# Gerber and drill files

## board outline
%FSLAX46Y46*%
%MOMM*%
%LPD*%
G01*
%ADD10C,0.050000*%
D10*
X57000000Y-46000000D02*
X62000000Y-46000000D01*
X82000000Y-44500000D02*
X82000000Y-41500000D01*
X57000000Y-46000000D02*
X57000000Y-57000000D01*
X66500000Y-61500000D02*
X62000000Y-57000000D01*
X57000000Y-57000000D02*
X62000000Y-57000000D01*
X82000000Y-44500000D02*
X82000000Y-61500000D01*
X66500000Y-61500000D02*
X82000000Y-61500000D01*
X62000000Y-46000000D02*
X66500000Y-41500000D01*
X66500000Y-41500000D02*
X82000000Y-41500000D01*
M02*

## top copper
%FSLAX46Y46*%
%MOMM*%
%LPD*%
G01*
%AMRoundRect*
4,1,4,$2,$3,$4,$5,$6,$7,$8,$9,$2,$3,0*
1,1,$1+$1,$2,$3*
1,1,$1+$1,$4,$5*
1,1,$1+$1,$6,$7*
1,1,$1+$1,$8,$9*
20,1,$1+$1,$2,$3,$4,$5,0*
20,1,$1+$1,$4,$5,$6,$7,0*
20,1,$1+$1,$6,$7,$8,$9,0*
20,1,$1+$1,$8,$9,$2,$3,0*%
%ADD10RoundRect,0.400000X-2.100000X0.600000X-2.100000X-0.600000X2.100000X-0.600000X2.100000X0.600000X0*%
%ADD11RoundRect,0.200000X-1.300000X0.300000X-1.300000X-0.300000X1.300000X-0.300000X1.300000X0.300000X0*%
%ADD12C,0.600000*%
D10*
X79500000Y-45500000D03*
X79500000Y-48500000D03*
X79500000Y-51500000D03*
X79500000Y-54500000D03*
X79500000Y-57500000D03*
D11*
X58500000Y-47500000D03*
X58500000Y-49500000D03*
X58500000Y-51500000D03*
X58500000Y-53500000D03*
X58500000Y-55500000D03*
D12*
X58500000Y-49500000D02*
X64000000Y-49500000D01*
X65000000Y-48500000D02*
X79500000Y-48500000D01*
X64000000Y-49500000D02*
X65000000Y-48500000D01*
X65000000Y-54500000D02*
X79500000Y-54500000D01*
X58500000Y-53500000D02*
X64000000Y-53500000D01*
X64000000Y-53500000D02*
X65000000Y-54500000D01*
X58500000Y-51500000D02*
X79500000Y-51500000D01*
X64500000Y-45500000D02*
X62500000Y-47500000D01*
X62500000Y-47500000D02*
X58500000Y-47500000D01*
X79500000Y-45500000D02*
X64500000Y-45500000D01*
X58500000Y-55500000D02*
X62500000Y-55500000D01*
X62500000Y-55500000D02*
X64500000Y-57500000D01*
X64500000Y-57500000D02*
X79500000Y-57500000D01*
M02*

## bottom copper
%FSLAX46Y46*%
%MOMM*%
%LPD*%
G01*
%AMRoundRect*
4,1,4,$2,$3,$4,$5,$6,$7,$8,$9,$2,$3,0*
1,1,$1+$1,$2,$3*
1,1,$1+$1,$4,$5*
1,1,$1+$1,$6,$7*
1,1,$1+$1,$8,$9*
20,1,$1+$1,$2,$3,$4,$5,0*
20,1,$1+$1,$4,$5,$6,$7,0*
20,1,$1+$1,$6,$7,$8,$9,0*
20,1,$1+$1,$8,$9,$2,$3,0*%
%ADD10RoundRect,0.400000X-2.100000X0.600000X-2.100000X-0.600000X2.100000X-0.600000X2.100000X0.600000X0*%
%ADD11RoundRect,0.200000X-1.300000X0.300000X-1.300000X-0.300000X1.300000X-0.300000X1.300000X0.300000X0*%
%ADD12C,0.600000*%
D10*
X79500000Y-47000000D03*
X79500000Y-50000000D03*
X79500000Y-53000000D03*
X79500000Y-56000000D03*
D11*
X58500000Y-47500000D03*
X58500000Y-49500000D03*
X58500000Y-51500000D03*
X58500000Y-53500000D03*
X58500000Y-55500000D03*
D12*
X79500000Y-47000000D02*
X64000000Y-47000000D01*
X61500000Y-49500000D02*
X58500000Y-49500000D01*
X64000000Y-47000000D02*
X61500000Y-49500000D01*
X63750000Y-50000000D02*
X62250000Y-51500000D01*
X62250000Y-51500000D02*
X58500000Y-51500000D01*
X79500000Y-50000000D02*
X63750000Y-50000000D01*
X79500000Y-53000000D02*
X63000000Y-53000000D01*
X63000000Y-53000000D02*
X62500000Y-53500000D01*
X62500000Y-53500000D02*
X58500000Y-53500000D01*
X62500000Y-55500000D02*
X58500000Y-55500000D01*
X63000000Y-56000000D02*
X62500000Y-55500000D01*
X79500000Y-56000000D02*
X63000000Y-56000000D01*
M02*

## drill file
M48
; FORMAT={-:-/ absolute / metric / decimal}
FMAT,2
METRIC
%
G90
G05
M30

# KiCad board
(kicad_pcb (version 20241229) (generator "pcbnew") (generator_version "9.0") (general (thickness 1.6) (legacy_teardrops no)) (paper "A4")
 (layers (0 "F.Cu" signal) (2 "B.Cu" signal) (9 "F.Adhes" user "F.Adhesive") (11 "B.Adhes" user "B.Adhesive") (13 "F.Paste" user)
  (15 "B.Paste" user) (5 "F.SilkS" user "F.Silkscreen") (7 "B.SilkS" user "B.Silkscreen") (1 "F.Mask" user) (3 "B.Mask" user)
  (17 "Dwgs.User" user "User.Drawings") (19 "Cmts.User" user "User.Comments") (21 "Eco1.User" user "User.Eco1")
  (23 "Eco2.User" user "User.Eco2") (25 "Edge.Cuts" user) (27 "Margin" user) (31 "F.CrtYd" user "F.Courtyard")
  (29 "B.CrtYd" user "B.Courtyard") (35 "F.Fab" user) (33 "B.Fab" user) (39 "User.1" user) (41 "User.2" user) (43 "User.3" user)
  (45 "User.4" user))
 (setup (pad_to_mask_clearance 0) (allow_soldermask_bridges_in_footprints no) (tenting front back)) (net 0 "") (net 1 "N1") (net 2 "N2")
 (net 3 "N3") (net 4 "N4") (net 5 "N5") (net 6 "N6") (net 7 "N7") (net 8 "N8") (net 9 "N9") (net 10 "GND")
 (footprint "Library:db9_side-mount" (layer "F.Cu") (at 79.5 51.5 -90)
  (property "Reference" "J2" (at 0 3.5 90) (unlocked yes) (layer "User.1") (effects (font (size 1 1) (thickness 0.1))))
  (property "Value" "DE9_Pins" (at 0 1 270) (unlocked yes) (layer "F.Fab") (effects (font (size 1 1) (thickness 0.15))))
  (pad "1" smd roundrect (at -6 0 270) (size 2 5) (layers "F.Cu" "F.Mask" "F.Paste") (roundrect_rratio 0.2) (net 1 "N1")
   (thermal_bridge_angle 45))
  (pad "2" smd roundrect (at -3 0 270) (size 2 5) (layers "F.Cu" "F.Mask" "F.Paste") (roundrect_rratio 0.2) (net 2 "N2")
   (thermal_bridge_angle 45))
  (pad "3" smd roundrect (at 0 0 270) (size 2 5) (layers "F.Cu" "F.Mask" "F.Paste") (roundrect_rratio 0.2) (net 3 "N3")
   (thermal_bridge_angle 45))
  (pad "4" smd roundrect (at 3 0 270) (size 2 5) (layers "F.Cu" "F.Mask" "F.Paste") (roundrect_rratio 0.2) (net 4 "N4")
   (thermal_bridge_angle 45))
  (pad "5" smd roundrect (at 6 0 270) (size 2 5) (layers "F.Cu" "F.Mask" "F.Paste") (roundrect_rratio 0.2) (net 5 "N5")
   (thermal_bridge_angle 45))
  (pad "6" smd roundrect (at -4.5 0 270) (size 2 5) (layers "B.Cu" "B.Mask" "B.Paste") (roundrect_rratio 0.2) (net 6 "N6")
   (thermal_bridge_angle 45))
  (pad "7" smd roundrect (at -1.5 0 270) (size 2 5) (layers "B.Cu" "B.Mask" "B.Paste") (roundrect_rratio 0.2) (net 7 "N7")
   (thermal_bridge_angle 45))
  (pad "8" smd roundrect (at 1.5 0 270) (size 2 5) (layers "B.Cu" "B.Mask" "B.Paste") (roundrect_rratio 0.2) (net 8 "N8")
   (thermal_bridge_angle 45))
  (pad "9" smd roundrect (at 4.5 0 270) (size 2 5) (layers "B.Cu" "B.Mask" "B.Paste") (roundrect_rratio 0.2) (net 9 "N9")
   (thermal_bridge_angle 45)))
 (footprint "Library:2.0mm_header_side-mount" (layer "B.Cu") (at 58.5 51.5 -90)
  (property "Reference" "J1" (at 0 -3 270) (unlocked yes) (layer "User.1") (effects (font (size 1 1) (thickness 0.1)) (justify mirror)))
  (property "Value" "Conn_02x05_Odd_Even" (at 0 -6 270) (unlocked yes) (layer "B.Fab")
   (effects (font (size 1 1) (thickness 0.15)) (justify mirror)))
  (pad "1" smd roundrect (at -4 0 270) (size 1 3) (layers "B.Cu" "B.Mask" "B.Paste") (roundrect_rratio 0.2) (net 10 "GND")
   (thermal_bridge_angle 45))
  (pad "2" smd roundrect (at -4 0 270) (size 1 3) (layers "F.Cu" "F.Mask" "F.Paste") (roundrect_rratio 0.2) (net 1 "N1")
   (thermal_bridge_angle 45))
  (pad "3" smd roundrect (at -2 0 270) (size 1 3) (layers "B.Cu" "B.Mask" "B.Paste") (roundrect_rratio 0.2) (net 6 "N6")
   (thermal_bridge_angle 45))
  (pad "4" smd roundrect (at -2 0 270) (size 1 3) (layers "F.Cu" "F.Mask" "F.Paste") (roundrect_rratio 0.2) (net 2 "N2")
   (thermal_bridge_angle 45))
  (pad "5" smd roundrect (at 0 0 270) (size 1 3) (layers "B.Cu" "B.Mask" "B.Paste") (roundrect_rratio 0.2) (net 7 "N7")
   (thermal_bridge_angle 45))
  (pad "6" smd roundrect (at 0 0 270) (size 1 3) (layers "F.Cu" "F.Mask" "F.Paste") (roundrect_rratio 0.2) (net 3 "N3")
   (thermal_bridge_angle 45))
  (pad "7" smd roundrect (at 2 0 270) (size 1 3) (layers "B.Cu" "B.Mask" "B.Paste") (roundrect_rratio 0.2) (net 8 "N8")
   (thermal_bridge_angle 45))
  (pad "8" smd roundrect (at 2 0 270) (size 1 3) (layers "F.Cu" "F.Mask" "F.Paste") (roundrect_rratio 0.2) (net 4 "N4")
   (thermal_bridge_angle 45))
  (pad "9" smd roundrect (at 4 0 270) (size 1 3) (layers "B.Cu" "B.Mask" "B.Paste") (roundrect_rratio 0.2) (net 9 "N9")
   (thermal_bridge_angle 45))
  (pad "10" smd roundrect (at 4 0 270) (size 1 3) (layers "F.Cu" "F.Mask" "F.Paste") (roundrect_rratio 0.2) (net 5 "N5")
   (thermal_bridge_angle 45)))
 (gr_line (start 57 46) (end 62 46) (stroke (width 0.05) (type default)) (layer "Edge.Cuts"))
 (gr_line (start 82 44.5) (end 82 41.5) (stroke (width 0.05) (type default)) (layer "Edge.Cuts"))
 (gr_line (start 57 46) (end 57 57) (stroke (width 0.05) (type default)) (layer "Edge.Cuts"))
 (gr_line (start 66.5 61.5) (end 62 57) (stroke (width 0.05) (type default)) (layer "Edge.Cuts"))
 (gr_line (start 57 57) (end 62 57) (stroke (width 0.05) (type default)) (layer "Edge.Cuts"))
 (gr_line (start 82 44.5) (end 82 61.5) (stroke (width 0.05) (type default)) (layer "Edge.Cuts"))
 (gr_line (start 66.5 61.5) (end 82 61.5) (stroke (width 0.05) (type default)) (layer "Edge.Cuts"))
 (gr_line (start 62 46) (end 66.5 41.5) (stroke (width 0.05) (type default)) (layer "Edge.Cuts"))
 (gr_line (start 66.5 41.5) (end 82 41.5) (stroke (width 0.05) (type default)) (layer "Edge.Cuts"))
 (segment (start 79.5 47) (end 64 47) (width 0.6) (layer "B.Cu") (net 6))
 (segment (start 61.5 49.5) (end 58.5 49.5) (width 0.6) (layer "B.Cu") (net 6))
 (segment (start 64 47) (end 61.5 49.5) (width 0.6) (layer "B.Cu") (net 6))
 (segment (start 58.5 49.5) (end 64 49.5) (width 0.6) (layer "F.Cu") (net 2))
 (segment (start 65 48.5) (end 79.5 48.5) (width 0.6) (layer "F.Cu") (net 2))
 (segment (start 64 49.5) (end 65 48.5) (width 0.6) (layer "F.Cu") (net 2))
 (segment (start 63.75 50) (end 62.25 51.5) (width 0.6) (layer "B.Cu") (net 7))
 (segment (start 62.25 51.5) (end 58.5 51.5) (width 0.6) (layer "B.Cu") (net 7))
 (segment (start 79.5 50) (end 63.75 50) (width 0.6) (layer "B.Cu") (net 7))
 (segment (start 65 54.5) (end 79.5 54.5) (width 0.6) (layer "F.Cu") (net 4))
 (segment (start 58.5 53.5) (end 64 53.5) (width 0.6) (layer "F.Cu") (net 4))
 (segment (start 64 53.5) (end 65 54.5) (width 0.6) (layer "F.Cu") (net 4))
 (segment (start 58.5 51.5) (end 79.5 51.5) (width 0.6) (layer "F.Cu") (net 3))
 (segment (start 79.5 53) (end 63 53) (width 0.6) (layer "B.Cu") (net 8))
 (segment (start 63 53) (end 62.5 53.5) (width 0.6) (layer "B.Cu") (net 8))
 (segment (start 62.5 53.5) (end 58.5 53.5) (width 0.6) (layer "B.Cu") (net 8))
 (segment (start 62.5 55.5) (end 58.5 55.5) (width 0.6) (layer "B.Cu") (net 9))
 (segment (start 63 56) (end 62.5 55.5) (width 0.6) (layer "B.Cu") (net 9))
 (segment (start 79.5 56) (end 63 56) (width 0.6) (layer "B.Cu") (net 9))
 (segment (start 64.5 45.5) (end 62.5 47.5) (width 0.6) (layer "F.Cu") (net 1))
 (segment (start 62.5 47.5) (end 58.5 47.5) (width 0.6) (layer "F.Cu") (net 1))
 (segment (start 79.5 45.5) (end 64.5 45.5) (width 0.6) (layer "F.Cu") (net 1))
 (segment (start 58.5 55.5) (end 62.5 55.5) (width 0.6) (layer "F.Cu") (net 5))
 (segment (start 62.5 55.5) (end 64.5 57.5) (width 0.6) (layer "F.Cu") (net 5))
 (segment (start 64.5 57.5) (end 79.5 57.5) (width 0.6) (layer "F.Cu") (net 5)))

